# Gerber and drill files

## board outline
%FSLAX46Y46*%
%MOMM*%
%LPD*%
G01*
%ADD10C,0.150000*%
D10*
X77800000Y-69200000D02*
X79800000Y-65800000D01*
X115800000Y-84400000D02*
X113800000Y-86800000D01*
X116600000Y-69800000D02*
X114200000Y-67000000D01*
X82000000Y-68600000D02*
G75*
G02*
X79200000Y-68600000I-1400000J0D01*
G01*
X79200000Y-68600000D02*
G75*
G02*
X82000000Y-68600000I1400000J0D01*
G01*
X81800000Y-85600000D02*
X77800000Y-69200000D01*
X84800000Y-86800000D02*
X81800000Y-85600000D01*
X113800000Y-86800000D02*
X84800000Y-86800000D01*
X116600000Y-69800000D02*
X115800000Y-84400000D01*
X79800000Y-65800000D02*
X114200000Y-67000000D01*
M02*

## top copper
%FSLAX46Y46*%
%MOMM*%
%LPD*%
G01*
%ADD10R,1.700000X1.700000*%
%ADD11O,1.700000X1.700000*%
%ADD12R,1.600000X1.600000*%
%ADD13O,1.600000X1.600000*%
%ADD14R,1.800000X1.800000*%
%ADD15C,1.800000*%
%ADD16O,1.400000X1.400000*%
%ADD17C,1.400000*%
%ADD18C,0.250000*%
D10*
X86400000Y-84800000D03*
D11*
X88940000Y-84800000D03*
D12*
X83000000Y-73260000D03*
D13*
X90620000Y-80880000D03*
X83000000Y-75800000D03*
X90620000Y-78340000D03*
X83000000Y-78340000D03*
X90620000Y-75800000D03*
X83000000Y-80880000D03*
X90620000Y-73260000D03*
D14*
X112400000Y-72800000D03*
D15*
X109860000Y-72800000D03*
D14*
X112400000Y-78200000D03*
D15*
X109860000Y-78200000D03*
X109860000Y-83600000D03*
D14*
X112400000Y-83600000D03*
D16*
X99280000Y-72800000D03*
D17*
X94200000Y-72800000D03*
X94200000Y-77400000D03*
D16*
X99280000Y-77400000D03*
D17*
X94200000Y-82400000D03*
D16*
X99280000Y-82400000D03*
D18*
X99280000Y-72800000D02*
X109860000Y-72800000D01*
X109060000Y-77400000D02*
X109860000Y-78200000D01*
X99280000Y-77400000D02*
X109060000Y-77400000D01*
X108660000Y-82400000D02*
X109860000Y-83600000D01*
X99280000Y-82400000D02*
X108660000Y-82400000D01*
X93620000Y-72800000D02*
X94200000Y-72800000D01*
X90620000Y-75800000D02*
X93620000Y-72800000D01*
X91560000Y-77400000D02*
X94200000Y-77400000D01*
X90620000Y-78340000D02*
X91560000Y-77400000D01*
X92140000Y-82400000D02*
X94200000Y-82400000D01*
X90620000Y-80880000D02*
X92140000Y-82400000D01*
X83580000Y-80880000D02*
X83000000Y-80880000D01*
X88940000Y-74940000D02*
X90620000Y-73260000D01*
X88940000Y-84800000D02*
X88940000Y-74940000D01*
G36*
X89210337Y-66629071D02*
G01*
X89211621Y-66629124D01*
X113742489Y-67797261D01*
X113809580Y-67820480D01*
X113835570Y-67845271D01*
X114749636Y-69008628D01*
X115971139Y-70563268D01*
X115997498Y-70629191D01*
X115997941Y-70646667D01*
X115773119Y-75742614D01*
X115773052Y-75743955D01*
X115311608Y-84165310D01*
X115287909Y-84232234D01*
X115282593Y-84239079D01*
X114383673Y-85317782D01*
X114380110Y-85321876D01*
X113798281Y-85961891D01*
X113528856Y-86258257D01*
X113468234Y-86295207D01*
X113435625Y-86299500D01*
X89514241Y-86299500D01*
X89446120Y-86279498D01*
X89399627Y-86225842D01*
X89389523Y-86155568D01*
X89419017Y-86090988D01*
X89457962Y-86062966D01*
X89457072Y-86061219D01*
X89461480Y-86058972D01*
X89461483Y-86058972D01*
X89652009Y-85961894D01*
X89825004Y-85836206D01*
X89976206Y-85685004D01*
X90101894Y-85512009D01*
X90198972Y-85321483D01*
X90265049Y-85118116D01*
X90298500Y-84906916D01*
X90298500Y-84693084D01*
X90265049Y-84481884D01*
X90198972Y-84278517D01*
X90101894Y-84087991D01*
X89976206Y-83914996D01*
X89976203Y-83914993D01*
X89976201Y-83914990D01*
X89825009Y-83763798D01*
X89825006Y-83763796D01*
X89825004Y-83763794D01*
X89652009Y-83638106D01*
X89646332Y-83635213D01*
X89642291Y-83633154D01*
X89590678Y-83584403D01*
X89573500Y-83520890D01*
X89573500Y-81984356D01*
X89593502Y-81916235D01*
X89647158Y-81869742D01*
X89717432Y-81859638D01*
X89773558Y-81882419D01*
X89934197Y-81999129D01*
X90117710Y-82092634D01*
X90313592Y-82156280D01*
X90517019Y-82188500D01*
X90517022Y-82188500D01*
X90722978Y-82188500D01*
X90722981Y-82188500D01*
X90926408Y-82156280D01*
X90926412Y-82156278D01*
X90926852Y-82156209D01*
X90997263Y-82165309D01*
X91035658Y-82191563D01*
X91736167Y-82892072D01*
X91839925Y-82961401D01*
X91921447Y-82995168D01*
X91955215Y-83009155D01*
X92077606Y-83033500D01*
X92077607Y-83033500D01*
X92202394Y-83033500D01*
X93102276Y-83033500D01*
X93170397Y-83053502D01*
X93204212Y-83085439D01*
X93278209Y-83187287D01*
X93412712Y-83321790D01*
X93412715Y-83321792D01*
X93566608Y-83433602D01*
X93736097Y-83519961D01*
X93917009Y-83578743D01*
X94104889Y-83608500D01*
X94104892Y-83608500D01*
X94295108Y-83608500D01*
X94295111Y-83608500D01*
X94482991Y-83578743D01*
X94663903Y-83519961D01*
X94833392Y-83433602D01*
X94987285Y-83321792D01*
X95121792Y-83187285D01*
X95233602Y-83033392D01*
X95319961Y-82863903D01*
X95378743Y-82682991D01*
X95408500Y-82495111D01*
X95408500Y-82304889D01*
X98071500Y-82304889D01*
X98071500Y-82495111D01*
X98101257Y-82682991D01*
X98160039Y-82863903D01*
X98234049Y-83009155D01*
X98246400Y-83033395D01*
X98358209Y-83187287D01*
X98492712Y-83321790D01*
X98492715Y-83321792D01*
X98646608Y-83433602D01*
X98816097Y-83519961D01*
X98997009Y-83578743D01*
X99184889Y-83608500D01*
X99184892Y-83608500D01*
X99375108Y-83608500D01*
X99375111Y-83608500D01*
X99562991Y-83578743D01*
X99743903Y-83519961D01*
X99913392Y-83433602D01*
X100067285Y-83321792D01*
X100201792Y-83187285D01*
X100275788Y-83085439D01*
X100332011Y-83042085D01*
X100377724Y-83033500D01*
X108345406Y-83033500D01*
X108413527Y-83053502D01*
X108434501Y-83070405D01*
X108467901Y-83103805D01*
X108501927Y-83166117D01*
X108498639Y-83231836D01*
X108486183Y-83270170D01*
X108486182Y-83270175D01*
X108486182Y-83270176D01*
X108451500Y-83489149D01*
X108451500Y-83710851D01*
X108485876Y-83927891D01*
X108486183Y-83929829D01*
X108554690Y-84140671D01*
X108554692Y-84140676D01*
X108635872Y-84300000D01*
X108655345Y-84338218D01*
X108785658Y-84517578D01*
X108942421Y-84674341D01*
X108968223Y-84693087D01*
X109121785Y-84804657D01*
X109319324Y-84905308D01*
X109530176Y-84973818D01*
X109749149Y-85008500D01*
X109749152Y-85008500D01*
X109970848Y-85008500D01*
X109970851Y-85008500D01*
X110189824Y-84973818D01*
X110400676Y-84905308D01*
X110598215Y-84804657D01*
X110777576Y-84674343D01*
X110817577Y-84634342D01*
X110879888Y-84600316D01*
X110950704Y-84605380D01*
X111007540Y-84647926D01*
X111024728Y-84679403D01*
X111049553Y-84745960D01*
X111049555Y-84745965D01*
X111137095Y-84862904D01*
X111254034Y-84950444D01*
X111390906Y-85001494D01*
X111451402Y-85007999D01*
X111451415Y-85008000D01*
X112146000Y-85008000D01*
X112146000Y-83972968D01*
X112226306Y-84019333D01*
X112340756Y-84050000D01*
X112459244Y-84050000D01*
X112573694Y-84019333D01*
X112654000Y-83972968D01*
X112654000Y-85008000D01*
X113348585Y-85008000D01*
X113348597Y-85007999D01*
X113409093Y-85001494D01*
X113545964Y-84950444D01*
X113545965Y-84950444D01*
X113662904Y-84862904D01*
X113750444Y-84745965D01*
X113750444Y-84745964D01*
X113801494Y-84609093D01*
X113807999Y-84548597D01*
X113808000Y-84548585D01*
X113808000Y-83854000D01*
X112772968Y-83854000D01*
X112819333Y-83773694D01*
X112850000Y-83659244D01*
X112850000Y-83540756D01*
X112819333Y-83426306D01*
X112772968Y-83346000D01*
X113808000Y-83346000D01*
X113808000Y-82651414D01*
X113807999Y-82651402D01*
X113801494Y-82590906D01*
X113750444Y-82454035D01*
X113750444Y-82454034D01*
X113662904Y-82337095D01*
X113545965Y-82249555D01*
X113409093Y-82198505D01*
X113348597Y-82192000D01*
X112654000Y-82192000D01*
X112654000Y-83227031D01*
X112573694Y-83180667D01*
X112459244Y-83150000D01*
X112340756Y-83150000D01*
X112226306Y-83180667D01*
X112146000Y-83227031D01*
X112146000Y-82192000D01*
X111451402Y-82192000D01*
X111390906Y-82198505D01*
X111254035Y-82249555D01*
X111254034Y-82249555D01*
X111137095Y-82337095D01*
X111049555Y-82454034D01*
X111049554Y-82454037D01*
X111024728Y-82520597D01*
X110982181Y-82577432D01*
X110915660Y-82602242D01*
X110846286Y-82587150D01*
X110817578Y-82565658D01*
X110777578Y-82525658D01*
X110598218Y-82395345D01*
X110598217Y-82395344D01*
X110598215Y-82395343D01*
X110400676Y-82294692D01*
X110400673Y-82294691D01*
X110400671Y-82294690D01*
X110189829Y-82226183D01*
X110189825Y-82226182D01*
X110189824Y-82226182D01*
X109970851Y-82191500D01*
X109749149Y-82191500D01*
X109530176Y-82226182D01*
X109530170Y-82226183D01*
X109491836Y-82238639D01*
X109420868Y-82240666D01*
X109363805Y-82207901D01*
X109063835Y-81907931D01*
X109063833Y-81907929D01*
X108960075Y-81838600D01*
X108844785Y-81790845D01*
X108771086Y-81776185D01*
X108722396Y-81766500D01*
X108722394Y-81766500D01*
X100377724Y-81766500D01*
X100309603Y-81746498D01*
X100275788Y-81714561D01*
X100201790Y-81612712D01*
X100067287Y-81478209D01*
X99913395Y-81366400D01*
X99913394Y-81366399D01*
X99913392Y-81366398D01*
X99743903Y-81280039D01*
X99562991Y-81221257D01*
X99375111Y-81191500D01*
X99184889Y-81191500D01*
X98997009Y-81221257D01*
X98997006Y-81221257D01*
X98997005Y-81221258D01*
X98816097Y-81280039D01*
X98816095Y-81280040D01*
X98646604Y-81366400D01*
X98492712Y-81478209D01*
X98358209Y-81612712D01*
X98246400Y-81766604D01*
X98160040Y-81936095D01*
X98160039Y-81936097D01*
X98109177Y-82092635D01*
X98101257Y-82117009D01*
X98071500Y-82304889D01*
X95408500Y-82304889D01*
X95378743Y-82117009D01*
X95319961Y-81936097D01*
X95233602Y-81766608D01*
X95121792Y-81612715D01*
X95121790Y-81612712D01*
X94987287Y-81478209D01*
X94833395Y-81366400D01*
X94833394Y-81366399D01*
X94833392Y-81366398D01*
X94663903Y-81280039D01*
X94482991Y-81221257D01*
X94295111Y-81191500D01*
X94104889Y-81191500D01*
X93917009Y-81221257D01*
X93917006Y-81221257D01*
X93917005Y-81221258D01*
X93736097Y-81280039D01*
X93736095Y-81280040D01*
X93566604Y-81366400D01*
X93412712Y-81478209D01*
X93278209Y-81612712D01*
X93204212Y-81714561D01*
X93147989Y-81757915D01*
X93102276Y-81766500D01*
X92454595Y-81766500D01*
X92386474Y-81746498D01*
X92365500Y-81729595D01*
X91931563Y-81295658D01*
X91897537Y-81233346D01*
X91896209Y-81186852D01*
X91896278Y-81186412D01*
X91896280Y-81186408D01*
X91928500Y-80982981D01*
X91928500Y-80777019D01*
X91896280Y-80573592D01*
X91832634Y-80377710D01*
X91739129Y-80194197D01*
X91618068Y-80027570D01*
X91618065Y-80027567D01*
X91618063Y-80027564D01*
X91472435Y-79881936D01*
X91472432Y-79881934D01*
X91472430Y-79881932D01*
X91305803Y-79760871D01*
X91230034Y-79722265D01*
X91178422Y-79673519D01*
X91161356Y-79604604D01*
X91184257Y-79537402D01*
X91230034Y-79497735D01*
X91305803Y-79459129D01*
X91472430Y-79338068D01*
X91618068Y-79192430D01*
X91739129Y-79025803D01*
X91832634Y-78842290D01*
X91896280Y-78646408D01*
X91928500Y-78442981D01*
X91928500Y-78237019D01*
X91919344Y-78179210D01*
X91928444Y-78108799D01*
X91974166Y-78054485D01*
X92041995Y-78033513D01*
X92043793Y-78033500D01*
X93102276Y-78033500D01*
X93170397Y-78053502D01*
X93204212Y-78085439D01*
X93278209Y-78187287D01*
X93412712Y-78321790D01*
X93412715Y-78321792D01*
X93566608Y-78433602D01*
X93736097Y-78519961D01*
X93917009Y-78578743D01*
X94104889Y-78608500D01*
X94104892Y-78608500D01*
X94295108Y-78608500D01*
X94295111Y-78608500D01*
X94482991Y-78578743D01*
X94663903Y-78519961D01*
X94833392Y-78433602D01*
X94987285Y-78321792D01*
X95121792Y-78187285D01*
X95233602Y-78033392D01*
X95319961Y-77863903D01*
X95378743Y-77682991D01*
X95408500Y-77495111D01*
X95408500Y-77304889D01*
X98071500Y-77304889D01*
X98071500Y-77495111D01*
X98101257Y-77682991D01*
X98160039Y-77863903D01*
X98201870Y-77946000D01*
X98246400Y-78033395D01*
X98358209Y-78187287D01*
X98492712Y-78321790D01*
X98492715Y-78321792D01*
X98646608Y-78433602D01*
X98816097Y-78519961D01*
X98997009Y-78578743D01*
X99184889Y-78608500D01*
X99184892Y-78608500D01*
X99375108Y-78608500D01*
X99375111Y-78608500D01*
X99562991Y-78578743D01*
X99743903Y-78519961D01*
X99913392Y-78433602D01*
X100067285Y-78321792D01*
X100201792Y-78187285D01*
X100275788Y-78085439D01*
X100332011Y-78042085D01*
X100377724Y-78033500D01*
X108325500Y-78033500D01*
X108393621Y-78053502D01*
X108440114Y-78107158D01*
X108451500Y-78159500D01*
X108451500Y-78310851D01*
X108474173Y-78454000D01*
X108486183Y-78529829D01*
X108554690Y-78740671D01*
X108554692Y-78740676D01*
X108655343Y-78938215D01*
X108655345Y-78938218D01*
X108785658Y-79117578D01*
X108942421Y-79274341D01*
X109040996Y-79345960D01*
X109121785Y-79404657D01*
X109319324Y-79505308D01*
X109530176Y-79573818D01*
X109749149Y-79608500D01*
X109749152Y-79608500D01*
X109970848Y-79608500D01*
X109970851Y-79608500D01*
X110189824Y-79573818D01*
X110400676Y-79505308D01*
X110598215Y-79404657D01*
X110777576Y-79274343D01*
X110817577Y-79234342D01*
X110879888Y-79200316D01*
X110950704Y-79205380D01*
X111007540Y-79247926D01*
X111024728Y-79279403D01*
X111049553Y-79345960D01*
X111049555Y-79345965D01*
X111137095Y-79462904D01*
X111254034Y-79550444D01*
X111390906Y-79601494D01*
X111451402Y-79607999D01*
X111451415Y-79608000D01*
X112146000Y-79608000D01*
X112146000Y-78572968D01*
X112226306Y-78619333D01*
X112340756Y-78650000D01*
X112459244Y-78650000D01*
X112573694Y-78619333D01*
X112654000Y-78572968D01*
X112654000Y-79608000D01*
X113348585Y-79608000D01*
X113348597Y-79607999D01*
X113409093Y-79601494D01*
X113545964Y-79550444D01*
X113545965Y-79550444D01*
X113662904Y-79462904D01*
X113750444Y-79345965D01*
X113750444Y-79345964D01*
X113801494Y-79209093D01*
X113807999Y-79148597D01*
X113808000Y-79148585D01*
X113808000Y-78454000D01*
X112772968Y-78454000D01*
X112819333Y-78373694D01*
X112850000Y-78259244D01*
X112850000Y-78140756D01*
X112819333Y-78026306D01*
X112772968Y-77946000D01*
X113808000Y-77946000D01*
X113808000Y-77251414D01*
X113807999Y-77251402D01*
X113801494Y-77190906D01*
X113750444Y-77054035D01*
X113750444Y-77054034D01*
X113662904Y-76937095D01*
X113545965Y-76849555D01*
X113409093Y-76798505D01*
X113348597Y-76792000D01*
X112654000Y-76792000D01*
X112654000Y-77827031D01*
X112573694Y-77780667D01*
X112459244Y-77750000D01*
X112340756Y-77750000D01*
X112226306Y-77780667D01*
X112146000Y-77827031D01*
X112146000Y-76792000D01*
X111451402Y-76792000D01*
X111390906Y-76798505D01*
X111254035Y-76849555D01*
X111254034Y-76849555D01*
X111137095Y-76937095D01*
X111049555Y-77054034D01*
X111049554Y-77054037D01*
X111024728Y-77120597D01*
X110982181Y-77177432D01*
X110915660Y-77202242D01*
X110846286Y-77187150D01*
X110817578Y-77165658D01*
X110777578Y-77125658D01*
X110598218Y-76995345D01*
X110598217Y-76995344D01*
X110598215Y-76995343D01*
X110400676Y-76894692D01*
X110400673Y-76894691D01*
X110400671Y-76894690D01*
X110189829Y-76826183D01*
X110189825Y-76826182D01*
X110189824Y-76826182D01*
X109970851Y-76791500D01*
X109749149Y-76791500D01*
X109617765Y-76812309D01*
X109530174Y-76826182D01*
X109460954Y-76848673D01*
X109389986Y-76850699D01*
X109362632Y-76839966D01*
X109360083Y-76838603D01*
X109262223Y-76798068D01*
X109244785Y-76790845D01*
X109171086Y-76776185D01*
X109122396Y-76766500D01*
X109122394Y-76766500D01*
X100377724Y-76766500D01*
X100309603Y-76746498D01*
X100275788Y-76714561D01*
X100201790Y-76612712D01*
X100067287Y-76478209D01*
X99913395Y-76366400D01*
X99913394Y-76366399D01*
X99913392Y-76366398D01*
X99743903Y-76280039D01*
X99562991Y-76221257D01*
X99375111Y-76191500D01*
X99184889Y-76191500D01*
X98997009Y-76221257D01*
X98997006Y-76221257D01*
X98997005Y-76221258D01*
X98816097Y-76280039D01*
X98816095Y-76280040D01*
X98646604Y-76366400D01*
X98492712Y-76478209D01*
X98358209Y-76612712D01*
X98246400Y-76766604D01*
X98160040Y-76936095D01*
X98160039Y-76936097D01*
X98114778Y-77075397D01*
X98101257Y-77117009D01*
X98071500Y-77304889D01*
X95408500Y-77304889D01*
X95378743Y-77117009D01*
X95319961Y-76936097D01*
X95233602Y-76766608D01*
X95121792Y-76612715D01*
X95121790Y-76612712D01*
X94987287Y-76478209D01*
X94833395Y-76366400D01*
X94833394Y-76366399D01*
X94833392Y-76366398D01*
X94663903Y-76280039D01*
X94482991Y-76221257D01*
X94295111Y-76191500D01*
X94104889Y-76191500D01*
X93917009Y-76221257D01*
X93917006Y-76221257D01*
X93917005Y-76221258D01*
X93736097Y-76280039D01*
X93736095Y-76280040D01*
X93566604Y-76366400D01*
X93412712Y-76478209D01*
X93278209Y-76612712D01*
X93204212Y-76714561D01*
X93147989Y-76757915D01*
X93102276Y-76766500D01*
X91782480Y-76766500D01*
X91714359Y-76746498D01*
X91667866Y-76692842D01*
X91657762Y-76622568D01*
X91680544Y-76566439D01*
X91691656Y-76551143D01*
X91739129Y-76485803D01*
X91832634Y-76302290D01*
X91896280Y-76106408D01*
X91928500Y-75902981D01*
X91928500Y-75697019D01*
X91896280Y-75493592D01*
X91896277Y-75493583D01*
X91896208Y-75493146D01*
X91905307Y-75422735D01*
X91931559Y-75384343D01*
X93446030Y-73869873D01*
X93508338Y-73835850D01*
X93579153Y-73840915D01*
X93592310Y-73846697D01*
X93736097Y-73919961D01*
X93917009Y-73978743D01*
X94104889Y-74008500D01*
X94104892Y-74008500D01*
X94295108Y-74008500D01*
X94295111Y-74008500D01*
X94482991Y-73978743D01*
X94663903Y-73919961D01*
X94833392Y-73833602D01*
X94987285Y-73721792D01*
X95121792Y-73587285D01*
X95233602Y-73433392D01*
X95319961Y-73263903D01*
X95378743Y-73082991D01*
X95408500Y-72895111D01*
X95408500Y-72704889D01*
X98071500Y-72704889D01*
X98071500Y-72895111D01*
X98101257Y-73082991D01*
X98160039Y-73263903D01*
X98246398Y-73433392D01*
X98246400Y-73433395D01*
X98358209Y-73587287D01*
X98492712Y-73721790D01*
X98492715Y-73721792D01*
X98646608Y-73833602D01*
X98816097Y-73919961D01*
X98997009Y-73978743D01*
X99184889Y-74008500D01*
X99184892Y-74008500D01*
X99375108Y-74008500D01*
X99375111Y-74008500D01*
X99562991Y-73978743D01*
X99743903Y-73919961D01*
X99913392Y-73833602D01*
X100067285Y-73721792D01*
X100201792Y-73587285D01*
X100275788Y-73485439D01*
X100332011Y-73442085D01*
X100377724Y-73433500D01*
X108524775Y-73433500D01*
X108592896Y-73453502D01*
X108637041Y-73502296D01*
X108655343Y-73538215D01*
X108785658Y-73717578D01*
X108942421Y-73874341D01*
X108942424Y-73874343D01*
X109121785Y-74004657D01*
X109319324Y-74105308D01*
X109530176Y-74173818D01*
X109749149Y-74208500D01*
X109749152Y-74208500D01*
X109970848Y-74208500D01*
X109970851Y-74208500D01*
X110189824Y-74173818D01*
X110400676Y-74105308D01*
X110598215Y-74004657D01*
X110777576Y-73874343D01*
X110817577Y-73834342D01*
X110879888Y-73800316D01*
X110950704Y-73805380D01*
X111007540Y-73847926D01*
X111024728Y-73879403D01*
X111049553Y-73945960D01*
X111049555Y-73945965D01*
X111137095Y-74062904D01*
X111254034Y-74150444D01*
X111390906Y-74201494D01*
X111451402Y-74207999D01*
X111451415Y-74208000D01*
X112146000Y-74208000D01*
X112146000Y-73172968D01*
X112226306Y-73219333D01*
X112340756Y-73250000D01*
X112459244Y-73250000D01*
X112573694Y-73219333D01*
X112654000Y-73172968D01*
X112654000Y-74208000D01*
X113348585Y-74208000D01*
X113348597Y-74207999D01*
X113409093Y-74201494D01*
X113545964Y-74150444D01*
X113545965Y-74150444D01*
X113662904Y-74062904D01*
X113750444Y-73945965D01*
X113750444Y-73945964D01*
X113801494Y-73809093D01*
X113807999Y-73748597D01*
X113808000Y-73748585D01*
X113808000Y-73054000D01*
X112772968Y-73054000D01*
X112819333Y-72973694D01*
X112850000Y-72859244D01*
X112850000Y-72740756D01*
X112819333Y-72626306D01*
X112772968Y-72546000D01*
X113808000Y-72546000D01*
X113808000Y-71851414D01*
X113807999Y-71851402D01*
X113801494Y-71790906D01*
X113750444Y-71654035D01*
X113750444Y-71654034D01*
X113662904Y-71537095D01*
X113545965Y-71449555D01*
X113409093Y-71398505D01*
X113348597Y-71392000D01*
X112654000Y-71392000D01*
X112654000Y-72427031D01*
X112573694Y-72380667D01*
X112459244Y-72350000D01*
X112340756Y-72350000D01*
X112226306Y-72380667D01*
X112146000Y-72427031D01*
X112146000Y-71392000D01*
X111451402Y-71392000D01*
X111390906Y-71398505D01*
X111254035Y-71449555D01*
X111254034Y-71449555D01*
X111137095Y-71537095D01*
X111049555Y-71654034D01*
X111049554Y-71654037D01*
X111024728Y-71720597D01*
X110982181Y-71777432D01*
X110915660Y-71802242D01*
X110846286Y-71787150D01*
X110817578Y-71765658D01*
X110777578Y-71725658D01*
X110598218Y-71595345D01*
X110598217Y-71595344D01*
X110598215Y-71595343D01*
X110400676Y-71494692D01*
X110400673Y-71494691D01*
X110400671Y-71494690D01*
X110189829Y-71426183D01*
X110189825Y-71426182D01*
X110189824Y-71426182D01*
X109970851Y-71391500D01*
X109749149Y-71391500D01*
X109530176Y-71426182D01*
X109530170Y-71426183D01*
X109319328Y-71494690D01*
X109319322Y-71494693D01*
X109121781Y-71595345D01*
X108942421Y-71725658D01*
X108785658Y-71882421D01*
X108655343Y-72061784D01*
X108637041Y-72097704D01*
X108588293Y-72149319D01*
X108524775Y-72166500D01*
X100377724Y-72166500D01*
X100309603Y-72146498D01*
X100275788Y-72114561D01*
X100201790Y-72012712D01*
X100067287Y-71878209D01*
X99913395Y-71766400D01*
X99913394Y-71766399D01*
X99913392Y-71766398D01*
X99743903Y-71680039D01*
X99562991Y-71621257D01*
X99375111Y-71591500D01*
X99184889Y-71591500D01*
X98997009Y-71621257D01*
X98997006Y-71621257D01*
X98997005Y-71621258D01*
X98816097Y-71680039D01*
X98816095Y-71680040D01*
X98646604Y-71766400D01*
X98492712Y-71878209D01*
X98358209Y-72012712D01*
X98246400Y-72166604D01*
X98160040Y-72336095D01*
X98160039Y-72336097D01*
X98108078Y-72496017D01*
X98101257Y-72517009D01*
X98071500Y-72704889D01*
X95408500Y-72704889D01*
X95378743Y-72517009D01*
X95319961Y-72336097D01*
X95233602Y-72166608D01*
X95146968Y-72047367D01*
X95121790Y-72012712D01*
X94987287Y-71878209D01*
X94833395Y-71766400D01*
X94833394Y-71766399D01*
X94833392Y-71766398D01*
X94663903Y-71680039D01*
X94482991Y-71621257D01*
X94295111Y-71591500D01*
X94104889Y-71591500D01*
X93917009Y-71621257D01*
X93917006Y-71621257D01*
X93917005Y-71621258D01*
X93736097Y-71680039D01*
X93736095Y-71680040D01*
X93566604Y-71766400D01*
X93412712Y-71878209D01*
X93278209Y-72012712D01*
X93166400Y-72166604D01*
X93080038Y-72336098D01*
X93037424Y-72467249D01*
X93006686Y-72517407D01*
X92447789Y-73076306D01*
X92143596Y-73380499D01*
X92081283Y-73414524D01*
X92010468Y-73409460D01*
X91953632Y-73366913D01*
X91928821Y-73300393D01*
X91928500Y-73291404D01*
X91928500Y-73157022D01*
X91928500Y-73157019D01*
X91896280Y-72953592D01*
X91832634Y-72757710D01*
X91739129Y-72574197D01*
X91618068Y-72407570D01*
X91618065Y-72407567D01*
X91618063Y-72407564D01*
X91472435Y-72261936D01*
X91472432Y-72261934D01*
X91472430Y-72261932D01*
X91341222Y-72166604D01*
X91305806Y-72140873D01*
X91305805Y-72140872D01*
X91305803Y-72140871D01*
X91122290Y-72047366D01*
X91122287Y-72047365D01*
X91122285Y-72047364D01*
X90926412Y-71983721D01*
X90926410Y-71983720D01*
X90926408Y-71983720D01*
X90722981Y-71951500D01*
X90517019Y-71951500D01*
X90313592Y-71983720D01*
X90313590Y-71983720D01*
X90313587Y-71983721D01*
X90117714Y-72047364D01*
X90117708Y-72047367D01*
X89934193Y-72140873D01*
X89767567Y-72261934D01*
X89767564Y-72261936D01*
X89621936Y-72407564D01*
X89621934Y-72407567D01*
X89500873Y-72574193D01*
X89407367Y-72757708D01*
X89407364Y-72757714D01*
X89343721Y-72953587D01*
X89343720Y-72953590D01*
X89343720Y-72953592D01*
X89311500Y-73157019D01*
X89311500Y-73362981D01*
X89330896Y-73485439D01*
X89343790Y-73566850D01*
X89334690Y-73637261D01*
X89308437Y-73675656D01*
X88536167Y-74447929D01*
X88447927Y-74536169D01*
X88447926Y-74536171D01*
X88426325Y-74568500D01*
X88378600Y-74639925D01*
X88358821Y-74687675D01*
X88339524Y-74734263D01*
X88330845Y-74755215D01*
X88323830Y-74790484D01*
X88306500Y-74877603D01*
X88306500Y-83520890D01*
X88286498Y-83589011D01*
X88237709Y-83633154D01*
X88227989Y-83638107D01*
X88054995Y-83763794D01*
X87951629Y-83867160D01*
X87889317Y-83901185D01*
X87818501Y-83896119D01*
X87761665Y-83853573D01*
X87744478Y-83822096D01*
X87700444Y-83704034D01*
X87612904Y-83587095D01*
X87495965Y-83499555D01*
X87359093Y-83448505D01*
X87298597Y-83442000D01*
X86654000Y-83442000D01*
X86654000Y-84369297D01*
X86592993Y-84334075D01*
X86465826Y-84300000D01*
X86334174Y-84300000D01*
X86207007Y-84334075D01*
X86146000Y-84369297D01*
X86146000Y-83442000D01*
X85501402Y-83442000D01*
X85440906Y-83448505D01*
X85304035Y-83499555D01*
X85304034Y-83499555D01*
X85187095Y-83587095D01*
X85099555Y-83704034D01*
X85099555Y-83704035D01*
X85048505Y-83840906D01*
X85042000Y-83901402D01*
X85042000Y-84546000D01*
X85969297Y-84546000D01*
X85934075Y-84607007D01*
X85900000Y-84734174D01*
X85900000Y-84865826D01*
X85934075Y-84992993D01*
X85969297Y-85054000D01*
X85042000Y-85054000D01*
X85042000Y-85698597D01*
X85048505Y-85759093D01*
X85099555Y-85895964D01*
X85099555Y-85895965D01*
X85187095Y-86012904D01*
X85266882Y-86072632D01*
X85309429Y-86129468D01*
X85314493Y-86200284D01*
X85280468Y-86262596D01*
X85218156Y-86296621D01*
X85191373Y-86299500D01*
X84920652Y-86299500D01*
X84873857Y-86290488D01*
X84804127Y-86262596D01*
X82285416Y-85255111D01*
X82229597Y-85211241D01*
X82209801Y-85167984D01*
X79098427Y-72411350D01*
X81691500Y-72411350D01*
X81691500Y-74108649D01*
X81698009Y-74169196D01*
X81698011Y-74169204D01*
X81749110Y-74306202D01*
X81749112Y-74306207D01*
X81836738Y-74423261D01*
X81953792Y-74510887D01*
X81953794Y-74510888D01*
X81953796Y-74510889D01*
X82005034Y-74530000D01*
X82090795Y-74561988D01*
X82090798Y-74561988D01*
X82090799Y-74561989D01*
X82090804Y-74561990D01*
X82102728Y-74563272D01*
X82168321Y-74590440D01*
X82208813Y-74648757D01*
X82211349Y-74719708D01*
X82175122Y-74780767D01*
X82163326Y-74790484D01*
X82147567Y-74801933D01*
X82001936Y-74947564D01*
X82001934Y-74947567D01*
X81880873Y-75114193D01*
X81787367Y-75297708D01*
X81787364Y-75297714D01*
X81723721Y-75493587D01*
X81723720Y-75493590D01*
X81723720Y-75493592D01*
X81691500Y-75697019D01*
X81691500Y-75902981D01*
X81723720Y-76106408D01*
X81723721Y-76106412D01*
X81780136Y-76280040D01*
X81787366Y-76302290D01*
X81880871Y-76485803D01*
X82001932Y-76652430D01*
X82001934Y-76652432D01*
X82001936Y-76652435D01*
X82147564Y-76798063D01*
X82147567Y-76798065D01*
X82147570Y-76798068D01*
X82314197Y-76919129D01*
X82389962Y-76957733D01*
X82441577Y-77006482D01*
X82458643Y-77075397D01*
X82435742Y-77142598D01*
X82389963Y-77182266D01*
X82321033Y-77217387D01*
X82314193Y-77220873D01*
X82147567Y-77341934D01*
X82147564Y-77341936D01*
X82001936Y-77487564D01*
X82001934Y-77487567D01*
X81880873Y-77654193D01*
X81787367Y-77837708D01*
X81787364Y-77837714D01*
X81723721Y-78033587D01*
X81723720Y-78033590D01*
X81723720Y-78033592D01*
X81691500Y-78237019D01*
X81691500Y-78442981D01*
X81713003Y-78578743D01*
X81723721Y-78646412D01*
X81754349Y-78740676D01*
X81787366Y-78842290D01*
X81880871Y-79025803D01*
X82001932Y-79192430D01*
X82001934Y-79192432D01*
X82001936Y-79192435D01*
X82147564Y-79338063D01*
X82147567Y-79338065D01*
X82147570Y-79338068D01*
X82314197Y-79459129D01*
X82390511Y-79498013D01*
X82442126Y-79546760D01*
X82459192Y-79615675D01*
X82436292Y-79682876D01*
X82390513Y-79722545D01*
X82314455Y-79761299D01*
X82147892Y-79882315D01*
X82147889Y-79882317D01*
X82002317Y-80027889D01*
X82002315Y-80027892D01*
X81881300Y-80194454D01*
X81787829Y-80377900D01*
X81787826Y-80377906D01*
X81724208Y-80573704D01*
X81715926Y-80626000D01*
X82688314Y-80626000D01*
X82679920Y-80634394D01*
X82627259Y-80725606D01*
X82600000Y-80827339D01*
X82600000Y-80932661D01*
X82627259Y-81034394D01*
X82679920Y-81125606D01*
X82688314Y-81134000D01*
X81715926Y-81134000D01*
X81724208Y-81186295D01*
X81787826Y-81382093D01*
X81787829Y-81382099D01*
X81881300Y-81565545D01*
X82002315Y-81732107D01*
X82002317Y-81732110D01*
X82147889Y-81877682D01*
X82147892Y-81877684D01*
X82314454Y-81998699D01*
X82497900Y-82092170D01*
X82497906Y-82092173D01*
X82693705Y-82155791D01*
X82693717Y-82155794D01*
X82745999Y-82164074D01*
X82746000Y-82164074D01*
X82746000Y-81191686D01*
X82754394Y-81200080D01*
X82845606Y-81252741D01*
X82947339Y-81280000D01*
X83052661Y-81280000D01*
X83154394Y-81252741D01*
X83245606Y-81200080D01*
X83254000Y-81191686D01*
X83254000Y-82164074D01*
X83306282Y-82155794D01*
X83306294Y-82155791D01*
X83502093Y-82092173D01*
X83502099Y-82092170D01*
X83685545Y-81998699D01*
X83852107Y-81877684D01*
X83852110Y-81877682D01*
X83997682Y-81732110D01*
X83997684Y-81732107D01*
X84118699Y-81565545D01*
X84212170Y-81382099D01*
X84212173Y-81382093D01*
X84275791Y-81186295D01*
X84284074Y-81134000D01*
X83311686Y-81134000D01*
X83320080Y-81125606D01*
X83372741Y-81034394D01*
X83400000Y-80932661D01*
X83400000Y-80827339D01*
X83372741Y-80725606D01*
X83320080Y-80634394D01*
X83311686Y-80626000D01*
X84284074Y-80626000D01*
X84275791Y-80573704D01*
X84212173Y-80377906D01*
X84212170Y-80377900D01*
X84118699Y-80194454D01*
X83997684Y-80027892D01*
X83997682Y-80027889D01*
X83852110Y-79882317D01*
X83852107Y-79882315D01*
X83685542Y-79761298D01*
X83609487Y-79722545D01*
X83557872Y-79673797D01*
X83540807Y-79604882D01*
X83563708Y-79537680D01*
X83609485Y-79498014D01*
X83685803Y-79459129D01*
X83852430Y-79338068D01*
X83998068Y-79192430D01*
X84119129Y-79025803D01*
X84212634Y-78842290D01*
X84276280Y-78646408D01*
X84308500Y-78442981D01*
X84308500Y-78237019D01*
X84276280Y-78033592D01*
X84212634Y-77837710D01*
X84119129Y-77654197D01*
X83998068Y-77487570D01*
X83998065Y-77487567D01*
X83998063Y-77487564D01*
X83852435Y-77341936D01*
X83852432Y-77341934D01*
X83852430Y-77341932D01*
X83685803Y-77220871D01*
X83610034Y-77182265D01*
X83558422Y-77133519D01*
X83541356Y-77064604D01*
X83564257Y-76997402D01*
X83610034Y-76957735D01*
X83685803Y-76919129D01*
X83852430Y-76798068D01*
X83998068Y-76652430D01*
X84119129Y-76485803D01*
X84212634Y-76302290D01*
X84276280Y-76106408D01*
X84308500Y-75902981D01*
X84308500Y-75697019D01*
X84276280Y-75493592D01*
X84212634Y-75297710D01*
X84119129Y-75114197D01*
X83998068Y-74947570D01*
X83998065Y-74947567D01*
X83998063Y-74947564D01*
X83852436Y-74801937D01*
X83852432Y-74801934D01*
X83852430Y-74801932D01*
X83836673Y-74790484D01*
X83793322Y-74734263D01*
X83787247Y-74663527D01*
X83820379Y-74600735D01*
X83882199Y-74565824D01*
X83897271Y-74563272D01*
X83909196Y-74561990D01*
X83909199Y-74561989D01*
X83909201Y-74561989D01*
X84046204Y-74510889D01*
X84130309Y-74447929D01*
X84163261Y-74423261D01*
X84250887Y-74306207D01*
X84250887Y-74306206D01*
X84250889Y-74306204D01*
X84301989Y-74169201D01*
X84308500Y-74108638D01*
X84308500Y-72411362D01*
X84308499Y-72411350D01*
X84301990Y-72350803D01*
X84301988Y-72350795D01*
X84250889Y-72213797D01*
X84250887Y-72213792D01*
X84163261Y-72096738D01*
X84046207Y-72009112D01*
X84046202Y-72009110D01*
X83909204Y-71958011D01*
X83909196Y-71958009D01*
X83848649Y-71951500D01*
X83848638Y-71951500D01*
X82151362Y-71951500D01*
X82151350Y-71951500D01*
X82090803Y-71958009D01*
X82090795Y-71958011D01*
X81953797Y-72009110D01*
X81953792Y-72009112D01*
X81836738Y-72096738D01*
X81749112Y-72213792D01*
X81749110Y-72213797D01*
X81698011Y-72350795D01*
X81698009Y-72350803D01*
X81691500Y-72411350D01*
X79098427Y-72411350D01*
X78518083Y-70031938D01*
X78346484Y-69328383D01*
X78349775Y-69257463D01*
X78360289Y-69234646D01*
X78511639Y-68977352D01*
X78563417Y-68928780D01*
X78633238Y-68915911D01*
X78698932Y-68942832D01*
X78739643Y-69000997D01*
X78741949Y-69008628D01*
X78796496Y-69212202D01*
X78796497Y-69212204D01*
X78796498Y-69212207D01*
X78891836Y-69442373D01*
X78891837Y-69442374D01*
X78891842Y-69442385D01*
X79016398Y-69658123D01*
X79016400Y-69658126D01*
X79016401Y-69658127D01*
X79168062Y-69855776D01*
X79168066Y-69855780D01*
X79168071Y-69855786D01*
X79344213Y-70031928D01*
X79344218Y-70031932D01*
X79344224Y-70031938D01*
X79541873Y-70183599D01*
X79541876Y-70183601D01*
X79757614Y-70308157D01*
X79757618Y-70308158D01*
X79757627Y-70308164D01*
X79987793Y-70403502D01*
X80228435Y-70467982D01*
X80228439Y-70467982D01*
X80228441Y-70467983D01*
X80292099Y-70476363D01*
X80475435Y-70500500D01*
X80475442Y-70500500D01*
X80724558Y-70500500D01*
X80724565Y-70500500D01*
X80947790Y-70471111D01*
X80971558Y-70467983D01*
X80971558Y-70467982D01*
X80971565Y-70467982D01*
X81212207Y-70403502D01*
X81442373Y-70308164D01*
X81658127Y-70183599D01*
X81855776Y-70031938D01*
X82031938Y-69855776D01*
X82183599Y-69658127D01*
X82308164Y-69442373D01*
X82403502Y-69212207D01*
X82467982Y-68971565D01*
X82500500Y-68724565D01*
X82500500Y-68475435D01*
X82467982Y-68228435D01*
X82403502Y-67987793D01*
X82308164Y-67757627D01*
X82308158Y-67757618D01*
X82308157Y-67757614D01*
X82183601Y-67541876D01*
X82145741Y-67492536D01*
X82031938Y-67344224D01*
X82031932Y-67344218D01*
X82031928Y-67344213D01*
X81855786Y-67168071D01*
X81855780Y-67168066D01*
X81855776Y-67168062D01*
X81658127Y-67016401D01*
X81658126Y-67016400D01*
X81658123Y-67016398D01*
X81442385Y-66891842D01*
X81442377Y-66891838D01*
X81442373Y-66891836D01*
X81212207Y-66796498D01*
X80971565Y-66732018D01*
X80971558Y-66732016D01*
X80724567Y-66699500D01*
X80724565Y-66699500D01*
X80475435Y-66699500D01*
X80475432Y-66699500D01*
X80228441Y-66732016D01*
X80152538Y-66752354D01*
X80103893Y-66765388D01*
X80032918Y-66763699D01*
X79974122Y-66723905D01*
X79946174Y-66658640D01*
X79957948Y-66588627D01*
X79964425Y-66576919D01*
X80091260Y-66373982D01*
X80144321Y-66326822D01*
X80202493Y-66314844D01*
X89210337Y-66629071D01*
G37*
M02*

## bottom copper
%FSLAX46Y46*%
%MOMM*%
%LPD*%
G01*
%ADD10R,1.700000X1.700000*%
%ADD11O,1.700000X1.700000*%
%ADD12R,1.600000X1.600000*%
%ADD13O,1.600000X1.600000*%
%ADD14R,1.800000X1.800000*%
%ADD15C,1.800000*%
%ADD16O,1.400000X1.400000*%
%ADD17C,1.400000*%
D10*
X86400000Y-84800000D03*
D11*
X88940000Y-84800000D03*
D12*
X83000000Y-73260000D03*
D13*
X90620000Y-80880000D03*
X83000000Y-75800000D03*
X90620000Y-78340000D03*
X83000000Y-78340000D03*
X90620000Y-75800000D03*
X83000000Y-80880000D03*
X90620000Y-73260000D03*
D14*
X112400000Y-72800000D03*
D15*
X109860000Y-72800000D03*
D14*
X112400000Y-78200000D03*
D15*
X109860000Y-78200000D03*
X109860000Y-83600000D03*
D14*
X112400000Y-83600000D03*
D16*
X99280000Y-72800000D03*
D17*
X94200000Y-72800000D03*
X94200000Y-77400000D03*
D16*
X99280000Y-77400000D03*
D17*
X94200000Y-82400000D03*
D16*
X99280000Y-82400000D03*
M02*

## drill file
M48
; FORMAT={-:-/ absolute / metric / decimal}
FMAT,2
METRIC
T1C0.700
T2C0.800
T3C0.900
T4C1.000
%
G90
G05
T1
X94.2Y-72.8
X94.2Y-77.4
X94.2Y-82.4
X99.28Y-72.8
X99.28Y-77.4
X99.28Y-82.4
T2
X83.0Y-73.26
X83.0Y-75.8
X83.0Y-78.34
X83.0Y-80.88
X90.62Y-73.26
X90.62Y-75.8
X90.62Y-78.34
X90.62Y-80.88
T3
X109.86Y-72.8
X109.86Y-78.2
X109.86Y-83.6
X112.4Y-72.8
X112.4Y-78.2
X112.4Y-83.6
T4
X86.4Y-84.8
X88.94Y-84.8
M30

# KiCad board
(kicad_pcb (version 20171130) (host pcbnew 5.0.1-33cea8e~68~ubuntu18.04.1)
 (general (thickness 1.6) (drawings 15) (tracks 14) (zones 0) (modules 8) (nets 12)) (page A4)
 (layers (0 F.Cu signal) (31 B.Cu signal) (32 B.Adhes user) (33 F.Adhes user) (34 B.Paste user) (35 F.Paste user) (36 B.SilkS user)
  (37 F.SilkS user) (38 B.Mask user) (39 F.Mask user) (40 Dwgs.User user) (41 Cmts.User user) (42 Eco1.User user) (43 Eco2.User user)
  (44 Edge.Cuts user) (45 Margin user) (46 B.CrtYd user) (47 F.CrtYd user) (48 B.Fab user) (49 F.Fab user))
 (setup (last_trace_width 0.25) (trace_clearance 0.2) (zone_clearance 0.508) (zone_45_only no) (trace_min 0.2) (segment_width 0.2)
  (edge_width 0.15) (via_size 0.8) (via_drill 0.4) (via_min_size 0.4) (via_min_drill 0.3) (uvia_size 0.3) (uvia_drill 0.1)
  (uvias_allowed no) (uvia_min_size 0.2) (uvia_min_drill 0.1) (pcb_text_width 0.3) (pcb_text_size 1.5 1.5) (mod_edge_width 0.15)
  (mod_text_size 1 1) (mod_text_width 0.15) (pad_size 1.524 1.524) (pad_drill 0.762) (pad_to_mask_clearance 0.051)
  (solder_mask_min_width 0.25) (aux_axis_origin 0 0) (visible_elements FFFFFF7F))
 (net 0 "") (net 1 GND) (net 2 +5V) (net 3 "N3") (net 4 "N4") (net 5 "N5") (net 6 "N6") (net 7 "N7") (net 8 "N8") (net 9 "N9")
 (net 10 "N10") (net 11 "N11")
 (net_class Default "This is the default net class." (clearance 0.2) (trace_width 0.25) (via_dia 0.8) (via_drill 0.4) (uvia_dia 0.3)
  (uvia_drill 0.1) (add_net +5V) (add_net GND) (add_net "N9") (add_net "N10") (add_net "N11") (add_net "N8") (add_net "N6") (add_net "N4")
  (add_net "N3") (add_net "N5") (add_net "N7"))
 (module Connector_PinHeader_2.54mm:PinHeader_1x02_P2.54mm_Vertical (layer F.Cu) (at 86.4 84.8 90)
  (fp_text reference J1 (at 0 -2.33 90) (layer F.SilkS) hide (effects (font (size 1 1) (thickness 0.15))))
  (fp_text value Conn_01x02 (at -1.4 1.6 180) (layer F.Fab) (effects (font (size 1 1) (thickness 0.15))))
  (pad 1 thru_hole rect (at 0 0 90) (size 1.7 1.7) (drill 1) (layers *.Cu *.Mask) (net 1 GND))
  (pad 2 thru_hole oval (at 0 2.54 90) (size 1.7 1.7) (drill 1) (layers *.Cu *.Mask) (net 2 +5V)))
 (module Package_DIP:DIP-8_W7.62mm (layer F.Cu) (at 83 73.26)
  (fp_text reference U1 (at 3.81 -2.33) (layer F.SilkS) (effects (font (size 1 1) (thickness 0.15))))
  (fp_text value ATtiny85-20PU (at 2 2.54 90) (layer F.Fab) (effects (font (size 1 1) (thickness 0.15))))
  (pad 1 thru_hole rect (at 0 0) (size 1.6 1.6) (drill 0.8) (layers *.Cu *.Mask) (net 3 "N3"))
  (pad 5 thru_hole oval (at 7.62 7.62) (size 1.6 1.6) (drill 0.8) (layers *.Cu *.Mask) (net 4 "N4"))
  (pad 2 thru_hole oval (at 0 2.54) (size 1.6 1.6) (drill 0.8) (layers *.Cu *.Mask) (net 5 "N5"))
  (pad 6 thru_hole oval (at 7.62 5.08) (size 1.6 1.6) (drill 0.8) (layers *.Cu *.Mask) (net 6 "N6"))
  (pad 3 thru_hole oval (at 0 5.08) (size 1.6 1.6) (drill 0.8) (layers *.Cu *.Mask) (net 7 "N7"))
  (pad 7 thru_hole oval (at 7.62 2.54) (size 1.6 1.6) (drill 0.8) (layers *.Cu *.Mask) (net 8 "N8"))
  (pad 4 thru_hole oval (at 0 7.62) (size 1.6 1.6) (drill 0.8) (layers *.Cu *.Mask) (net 1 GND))
  (pad 8 thru_hole oval (at 7.62 0) (size 1.6 1.6) (drill 0.8) (layers *.Cu *.Mask) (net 2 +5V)))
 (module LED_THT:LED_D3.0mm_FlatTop (layer F.Cu) (at 112.4 72.8 180)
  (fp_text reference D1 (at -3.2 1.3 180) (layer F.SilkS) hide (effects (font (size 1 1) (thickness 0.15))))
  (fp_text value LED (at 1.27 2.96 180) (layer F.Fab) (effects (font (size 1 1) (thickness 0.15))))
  (pad 1 thru_hole rect (at 0 0 180) (size 1.8 1.8) (drill 0.9) (layers *.Cu *.Mask) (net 1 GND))
  (pad 2 thru_hole circle (at 2.54 0 180) (size 1.8 1.8) (drill 0.9) (layers *.Cu *.Mask) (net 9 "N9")))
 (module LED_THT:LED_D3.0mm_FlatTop (layer F.Cu) (at 112.4 78.2 180)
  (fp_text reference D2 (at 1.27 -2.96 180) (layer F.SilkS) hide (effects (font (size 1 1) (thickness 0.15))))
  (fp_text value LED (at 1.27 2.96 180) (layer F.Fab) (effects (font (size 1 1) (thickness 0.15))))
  (pad 1 thru_hole rect (at 0 0 180) (size 1.8 1.8) (drill 0.9) (layers *.Cu *.Mask) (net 1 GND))
  (pad 2 thru_hole circle (at 2.54 0 180) (size 1.8 1.8) (drill 0.9) (layers *.Cu *.Mask) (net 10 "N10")))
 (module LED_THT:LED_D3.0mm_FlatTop (layer F.Cu) (at 112.4 83.6 180)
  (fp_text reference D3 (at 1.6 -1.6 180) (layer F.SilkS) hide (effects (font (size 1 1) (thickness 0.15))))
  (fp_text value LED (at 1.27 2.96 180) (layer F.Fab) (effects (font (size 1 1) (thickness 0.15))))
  (pad 2 thru_hole circle (at 2.54 0 180) (size 1.8 1.8) (drill 0.9) (layers *.Cu *.Mask) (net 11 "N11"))
  (pad 1 thru_hole rect (at 0 0 180) (size 1.8 1.8) (drill 0.9) (layers *.Cu *.Mask) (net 1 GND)))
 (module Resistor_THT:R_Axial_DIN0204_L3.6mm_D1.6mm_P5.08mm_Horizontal (layer F.Cu) (at 94.2 72.8)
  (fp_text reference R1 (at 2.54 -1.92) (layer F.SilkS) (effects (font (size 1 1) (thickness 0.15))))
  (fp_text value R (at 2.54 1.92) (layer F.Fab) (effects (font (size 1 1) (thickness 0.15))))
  (pad 2 thru_hole oval (at 5.08 0) (size 1.4 1.4) (drill 0.7) (layers *.Cu *.Mask) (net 9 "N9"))
  (pad 1 thru_hole circle (at 0 0) (size 1.4 1.4) (drill 0.7) (layers *.Cu *.Mask) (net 8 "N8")))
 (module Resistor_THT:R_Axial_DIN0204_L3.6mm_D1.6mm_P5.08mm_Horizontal (layer F.Cu) (at 94.2 77.4)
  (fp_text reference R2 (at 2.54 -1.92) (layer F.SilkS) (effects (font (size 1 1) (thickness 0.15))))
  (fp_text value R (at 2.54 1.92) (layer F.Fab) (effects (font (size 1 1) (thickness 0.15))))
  (pad 1 thru_hole circle (at 0 0) (size 1.4 1.4) (drill 0.7) (layers *.Cu *.Mask) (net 6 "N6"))
  (pad 2 thru_hole oval (at 5.08 0) (size 1.4 1.4) (drill 0.7) (layers *.Cu *.Mask) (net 10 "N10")))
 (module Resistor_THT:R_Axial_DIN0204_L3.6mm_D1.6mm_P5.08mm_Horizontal (layer F.Cu) (at 94.2 82.4)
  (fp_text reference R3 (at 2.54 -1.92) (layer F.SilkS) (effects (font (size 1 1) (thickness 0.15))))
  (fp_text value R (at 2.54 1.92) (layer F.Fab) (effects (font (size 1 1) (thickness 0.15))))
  (pad 1 thru_hole circle (at 0 0) (size 1.4 1.4) (drill 0.7) (layers *.Cu *.Mask) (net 4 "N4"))
  (pad 2 thru_hole oval (at 5.08 0) (size 1.4 1.4) (drill 0.7) (layers *.Cu *.Mask) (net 11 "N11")))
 (gr_line (start 77.8 69.2) (end 79.8 65.8) (layer Edge.Cuts) (width 0.15))
 (gr_line (start 115.8 84.4) (end 113.8 86.8) (layer Edge.Cuts) (width 0.15))
 (gr_line (start 116.6 69.8) (end 114.2 67) (layer Edge.Cuts) (width 0.15))
 (gr_circle (center 80.6 68.6) (end 82 68.6) (layer Edge.Cuts) (width 0.15))
 (gr_line (start 81.8 85.6) (end 77.8 69.2) (layer Edge.Cuts) (width 0.15))
 (gr_line (start 84.8 86.8) (end 81.8 85.6) (layer Edge.Cuts) (width 0.15))
 (gr_line (start 113.8 86.8) (end 84.8 86.8) (layer Edge.Cuts) (width 0.15))
 (gr_line (start 116.6 69.8) (end 115.8 84.4) (layer Edge.Cuts) (width 0.15))
 (gr_line (start 79.8 65.8) (end 114.2 67) (layer Edge.Cuts) (width 0.15))
 (segment (start 99.28 72.8) (end 109.86 72.8) (width 0.25) (layer F.Cu) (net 9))
 (segment (start 109.06 77.4) (end 109.86 78.2) (width 0.25) (layer F.Cu) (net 10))
 (segment (start 99.28 77.4) (end 109.06 77.4) (width 0.25) (layer F.Cu) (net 10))
 (segment (start 108.66 82.4) (end 109.86 83.6) (width 0.25) (layer F.Cu) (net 11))
 (segment (start 99.28 82.4) (end 108.66 82.4) (width 0.25) (layer F.Cu) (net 11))
 (segment (start 93.62 72.8) (end 94.2 72.8) (width 0.25) (layer F.Cu) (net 8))
 (segment (start 90.62 75.8) (end 93.62 72.8) (width 0.25) (layer F.Cu) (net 8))
 (segment (start 91.56 77.4) (end 94.2 77.4) (width 0.25) (layer F.Cu) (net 6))
 (segment (start 90.62 78.34) (end 91.56 77.4) (width 0.25) (layer F.Cu) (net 6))
 (segment (start 92.14 82.4) (end 94.2 82.4) (width 0.25) (layer F.Cu) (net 4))
 (segment (start 90.62 80.88) (end 92.14 82.4) (width 0.25) (layer F.Cu) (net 4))
 (segment (start 83.58 80.88) (end 83 80.88) (width 0.25) (layer F.Cu) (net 1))
 (segment (start 88.94 74.94) (end 90.62 73.26) (width 0.25) (layer F.Cu) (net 2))
 (segment (start 88.94 84.8) (end 88.94 74.94) (width 0.25) (layer F.Cu) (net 2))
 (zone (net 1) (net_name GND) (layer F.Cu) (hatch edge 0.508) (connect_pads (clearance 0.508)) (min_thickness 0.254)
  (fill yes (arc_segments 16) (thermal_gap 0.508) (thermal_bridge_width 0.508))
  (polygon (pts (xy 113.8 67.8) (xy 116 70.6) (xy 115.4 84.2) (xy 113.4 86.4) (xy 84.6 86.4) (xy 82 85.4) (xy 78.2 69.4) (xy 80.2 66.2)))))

